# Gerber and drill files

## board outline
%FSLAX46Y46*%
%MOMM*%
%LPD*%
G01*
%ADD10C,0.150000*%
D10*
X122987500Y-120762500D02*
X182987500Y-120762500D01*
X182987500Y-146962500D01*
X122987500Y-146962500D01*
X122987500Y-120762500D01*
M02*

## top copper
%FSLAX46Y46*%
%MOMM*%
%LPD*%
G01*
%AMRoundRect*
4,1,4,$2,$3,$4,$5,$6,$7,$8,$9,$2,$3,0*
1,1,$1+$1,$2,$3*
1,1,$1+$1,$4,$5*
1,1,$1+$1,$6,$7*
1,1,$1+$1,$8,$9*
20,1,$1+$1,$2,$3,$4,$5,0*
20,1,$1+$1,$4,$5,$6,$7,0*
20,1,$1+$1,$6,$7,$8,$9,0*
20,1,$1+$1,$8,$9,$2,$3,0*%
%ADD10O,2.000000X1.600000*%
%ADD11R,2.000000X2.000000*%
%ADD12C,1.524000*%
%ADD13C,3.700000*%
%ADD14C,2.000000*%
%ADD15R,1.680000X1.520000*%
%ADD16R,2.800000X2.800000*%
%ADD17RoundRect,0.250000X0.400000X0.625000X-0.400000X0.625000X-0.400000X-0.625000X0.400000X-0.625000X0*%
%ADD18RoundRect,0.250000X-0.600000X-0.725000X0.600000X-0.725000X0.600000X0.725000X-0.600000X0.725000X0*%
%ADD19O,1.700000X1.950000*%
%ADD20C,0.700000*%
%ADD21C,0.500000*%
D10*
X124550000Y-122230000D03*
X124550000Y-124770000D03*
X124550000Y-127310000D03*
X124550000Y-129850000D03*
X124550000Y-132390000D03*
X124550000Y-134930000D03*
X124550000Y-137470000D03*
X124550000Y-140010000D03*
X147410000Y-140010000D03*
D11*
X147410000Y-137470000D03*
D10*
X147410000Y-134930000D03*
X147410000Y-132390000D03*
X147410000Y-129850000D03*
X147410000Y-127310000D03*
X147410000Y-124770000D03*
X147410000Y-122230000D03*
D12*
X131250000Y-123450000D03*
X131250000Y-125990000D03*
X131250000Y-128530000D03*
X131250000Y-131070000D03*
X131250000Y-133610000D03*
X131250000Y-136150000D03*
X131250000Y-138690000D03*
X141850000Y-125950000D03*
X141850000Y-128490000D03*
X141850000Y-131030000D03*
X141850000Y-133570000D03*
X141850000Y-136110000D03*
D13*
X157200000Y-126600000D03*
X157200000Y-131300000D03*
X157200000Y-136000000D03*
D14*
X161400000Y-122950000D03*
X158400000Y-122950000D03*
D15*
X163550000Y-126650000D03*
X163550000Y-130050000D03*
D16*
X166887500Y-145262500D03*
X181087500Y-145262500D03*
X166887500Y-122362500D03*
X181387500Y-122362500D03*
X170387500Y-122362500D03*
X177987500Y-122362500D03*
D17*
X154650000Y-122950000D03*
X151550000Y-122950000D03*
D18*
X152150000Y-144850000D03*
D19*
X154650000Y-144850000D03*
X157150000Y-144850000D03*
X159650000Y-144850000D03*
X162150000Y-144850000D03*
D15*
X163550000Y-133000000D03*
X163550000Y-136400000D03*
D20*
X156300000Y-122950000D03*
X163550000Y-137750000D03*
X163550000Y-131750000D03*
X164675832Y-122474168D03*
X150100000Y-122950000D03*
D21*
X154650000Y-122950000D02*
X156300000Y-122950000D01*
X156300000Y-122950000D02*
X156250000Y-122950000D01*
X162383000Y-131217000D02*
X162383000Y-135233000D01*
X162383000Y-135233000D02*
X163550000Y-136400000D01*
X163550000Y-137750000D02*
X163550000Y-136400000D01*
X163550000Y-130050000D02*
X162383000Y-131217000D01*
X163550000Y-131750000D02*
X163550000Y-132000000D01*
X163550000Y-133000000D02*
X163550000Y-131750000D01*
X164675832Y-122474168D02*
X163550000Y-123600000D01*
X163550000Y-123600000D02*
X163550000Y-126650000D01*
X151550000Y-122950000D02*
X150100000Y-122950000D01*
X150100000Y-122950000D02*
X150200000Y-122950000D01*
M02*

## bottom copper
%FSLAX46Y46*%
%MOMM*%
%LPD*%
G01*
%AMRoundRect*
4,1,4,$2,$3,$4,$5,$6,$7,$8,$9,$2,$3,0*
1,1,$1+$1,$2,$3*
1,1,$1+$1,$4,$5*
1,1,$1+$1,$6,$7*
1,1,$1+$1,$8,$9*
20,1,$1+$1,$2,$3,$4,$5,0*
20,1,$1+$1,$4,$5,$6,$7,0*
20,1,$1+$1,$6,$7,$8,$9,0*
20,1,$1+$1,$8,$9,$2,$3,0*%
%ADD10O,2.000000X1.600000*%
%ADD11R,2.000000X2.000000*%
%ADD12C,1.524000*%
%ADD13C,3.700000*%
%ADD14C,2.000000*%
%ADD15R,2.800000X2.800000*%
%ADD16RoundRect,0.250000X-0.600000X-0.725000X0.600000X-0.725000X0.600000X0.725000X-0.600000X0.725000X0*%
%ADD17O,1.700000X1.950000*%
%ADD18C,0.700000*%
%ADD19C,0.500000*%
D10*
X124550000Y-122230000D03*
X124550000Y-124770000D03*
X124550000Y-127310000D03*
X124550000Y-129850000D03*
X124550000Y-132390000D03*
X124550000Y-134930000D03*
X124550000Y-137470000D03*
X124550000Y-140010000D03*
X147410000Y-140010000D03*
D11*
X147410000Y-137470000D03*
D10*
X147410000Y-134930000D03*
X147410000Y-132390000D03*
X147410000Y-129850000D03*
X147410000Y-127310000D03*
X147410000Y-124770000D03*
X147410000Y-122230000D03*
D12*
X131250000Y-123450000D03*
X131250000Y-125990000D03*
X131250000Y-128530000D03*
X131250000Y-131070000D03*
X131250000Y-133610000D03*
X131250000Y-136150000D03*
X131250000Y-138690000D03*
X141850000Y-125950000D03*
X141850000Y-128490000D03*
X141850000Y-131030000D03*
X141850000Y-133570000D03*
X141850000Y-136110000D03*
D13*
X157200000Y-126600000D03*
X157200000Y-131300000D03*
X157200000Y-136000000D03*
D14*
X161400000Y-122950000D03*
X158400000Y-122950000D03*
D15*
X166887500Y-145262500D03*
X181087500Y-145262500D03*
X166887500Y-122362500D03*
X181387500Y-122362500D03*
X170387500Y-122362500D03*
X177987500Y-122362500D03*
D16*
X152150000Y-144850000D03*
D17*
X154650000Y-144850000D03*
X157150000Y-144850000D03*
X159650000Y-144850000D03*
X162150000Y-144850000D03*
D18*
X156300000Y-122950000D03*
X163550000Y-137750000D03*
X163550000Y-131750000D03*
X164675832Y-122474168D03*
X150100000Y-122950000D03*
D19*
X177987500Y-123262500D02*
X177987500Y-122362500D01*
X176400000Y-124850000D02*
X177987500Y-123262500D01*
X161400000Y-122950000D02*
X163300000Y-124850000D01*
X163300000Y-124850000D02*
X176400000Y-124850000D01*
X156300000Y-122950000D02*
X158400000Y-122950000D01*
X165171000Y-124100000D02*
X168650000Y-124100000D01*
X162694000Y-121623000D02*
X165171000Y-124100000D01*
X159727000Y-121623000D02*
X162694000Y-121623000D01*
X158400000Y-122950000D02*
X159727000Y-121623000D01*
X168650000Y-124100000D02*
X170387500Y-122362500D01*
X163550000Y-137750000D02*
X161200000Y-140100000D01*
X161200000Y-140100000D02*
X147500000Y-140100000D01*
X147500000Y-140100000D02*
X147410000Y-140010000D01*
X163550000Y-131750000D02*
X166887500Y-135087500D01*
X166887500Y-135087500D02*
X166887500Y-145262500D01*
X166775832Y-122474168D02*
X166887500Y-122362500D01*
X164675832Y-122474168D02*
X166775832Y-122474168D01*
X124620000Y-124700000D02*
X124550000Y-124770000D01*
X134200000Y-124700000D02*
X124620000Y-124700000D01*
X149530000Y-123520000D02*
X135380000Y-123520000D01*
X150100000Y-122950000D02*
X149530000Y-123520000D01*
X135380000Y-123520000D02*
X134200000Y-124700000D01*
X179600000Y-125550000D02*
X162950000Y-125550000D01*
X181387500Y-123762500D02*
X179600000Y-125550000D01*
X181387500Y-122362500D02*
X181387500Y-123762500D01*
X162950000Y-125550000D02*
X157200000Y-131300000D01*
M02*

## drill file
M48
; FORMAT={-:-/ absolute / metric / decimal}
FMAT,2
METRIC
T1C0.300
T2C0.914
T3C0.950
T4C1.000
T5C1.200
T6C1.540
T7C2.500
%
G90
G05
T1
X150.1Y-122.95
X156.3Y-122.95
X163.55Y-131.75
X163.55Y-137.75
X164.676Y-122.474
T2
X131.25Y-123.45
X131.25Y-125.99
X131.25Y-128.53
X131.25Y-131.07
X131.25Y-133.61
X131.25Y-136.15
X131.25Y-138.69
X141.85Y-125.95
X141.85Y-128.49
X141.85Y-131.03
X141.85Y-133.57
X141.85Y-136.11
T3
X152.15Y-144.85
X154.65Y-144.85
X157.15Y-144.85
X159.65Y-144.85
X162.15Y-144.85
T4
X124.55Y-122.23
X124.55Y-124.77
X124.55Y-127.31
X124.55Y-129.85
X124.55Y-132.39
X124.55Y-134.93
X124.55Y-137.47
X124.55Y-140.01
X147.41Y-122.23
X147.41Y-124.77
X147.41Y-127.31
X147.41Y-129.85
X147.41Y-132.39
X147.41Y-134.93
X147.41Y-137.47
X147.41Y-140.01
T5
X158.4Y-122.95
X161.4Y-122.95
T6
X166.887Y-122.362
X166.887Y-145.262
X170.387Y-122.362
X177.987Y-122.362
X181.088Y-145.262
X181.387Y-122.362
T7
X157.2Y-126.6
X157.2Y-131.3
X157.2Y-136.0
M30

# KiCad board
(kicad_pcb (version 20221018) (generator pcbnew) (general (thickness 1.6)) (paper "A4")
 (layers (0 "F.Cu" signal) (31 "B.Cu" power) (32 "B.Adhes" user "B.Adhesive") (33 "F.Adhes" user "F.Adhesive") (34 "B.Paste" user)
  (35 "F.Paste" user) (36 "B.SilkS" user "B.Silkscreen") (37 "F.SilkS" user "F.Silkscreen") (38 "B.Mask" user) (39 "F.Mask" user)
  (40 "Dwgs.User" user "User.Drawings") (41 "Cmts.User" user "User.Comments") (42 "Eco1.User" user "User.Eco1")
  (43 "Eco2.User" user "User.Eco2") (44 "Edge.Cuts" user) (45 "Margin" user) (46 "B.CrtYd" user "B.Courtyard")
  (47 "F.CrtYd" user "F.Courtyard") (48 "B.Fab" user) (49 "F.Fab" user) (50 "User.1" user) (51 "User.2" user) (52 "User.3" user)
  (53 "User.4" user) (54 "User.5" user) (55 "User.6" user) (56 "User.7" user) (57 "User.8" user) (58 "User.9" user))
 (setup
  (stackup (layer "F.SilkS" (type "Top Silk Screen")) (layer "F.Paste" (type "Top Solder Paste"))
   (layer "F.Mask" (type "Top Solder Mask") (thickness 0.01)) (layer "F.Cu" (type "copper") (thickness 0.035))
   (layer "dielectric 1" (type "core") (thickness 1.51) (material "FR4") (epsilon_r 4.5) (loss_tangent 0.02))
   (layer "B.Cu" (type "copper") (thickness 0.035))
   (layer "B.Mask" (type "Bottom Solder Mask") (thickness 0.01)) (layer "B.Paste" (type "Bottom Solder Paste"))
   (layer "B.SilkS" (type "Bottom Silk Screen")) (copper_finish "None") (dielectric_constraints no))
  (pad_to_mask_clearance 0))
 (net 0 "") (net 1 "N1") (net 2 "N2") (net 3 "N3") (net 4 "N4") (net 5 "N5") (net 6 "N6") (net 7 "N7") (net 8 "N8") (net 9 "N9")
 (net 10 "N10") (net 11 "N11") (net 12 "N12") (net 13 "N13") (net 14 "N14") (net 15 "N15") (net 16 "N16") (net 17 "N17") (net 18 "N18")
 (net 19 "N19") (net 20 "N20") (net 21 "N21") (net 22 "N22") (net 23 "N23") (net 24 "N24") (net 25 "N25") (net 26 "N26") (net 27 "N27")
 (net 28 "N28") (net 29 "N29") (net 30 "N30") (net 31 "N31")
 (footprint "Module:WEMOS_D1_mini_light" (layer "F.Cu") (at 124.55 122.23)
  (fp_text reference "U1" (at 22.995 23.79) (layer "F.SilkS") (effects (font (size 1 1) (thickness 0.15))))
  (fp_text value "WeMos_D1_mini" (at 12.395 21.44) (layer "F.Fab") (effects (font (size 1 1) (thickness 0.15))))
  (pad "1" thru_hole oval (at 0 0) (size 2 1.6) (drill 1) (layers "*.Cu" "*.Mask") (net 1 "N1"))
  (pad "2" thru_hole oval (at 0 2.54) (size 2 1.6) (drill 1) (layers "*.Cu" "*.Mask") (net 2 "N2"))
  (pad "3" thru_hole oval (at 0 5.08) (size 2 1.6) (drill 1) (layers "*.Cu" "*.Mask") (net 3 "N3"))
  (pad "4" thru_hole oval (at 0 7.62) (size 2 1.6) (drill 1) (layers "*.Cu" "*.Mask") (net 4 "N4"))
  (pad "5" thru_hole oval (at 0 10.16) (size 2 1.6) (drill 1) (layers "*.Cu" "*.Mask") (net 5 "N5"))
  (pad "6" thru_hole oval (at 0 12.7) (size 2 1.6) (drill 1) (layers "*.Cu" "*.Mask") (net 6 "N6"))
  (pad "7" thru_hole oval (at 0 15.24) (size 2 1.6) (drill 1) (layers "*.Cu" "*.Mask") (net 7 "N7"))
  (pad "8" thru_hole oval (at 0 17.78) (size 2 1.6) (drill 1) (layers "*.Cu" "*.Mask") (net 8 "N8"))
  (pad "9" thru_hole oval (at 22.86 17.78) (size 2 1.6) (drill 1) (layers "*.Cu" "*.Mask") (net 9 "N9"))
  (pad "10" thru_hole rect (at 22.86 15.24) (size 2 2) (drill 1) (layers "*.Cu" "*.Mask") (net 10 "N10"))
  (pad "11" thru_hole oval (at 22.86 12.7) (size 2 1.6) (drill 1) (layers "*.Cu" "*.Mask") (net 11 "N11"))
  (pad "12" thru_hole oval (at 22.86 10.16) (size 2 1.6) (drill 1) (layers "*.Cu" "*.Mask") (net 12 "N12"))
  (pad "13" thru_hole oval (at 22.86 7.62) (size 2 1.6) (drill 1) (layers "*.Cu" "*.Mask") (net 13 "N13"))
  (pad "14" thru_hole oval (at 22.86 5.08) (size 2 1.6) (drill 1) (layers "*.Cu" "*.Mask") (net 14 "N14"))
  (pad "15" thru_hole oval (at 22.86 2.54) (size 2 1.6) (drill 1) (layers "*.Cu" "*.Mask") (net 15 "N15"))
  (pad "16" thru_hole oval (at 22.86 0) (size 2 1.6) (drill 1) (layers "*.Cu" "*.Mask") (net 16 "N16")))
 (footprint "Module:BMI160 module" (layer "F.Cu") (at 129.975 122.075)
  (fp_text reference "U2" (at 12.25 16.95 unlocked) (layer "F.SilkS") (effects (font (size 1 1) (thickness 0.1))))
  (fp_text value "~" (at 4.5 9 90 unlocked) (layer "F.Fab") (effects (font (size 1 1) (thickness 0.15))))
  (pad "1" thru_hole circle (at 1.275 1.375) (size 1.524 1.524) (drill 0.914) (layers "*.Cu" "*.Mask") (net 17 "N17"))
  (pad "2" thru_hole circle (at 1.275 3.915) (size 1.524 1.524) (drill 0.914) (layers "*.Cu" "*.Mask") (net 8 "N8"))
  (pad "3" thru_hole circle (at 1.275 6.455) (size 1.524 1.524) (drill 0.914) (layers "*.Cu" "*.Mask") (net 10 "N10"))
  (pad "4" thru_hole circle (at 1.275 8.995) (size 1.524 1.524) (drill 0.914) (layers "*.Cu" "*.Mask") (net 14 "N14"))
  (pad "5" thru_hole circle (at 1.275 11.535) (size 1.524 1.524) (drill 0.914) (layers "*.Cu" "*.Mask") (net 13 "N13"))
  (pad "6" thru_hole circle (at 1.275 14.075) (size 1.524 1.524) (drill 0.914) (layers "*.Cu" "*.Mask") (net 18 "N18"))
  (pad "7" thru_hole circle (at 1.275 16.615) (size 1.524 1.524) (drill 0.914) (layers "*.Cu" "*.Mask") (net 10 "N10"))
  (pad "8" thru_hole circle (at 11.875 3.875) (size 1.524 1.524) (drill 0.914) (layers "*.Cu" "*.Mask") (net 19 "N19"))
  (pad "9" thru_hole circle (at 11.875 6.415) (size 1.524 1.524) (drill 0.914) (layers "*.Cu" "*.Mask") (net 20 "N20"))
  (pad "10" thru_hole circle (at 11.875 8.955) (size 1.524 1.524) (drill 0.914) (layers "*.Cu" "*.Mask") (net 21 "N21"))
  (pad "11" thru_hole circle (at 11.875 11.495) (size 1.524 1.524) (drill 0.914) (layers "*.Cu" "*.Mask") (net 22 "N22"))
  (pad "12" thru_hole circle (at 11.875 14.035) (size 1.524 1.524) (drill 0.914) (layers "*.Cu" "*.Mask") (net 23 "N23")))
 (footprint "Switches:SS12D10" (layer "F.Cu") (at 157.1 131.25 -90)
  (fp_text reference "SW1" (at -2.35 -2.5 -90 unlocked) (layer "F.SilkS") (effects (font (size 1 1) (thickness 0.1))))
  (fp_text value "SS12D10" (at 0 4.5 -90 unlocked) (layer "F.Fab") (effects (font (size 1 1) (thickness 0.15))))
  (pad "1" thru_hole circle (at -4.65 -0.1 270) (size 3.7 3.7) (drill 2.5) (layers "*.Cu" "*.Mask") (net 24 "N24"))
  (pad "2" thru_hole circle (at 0.05 -0.1 270) (size 3.7 3.7) (drill 2.5) (layers "*.Cu" "*.Mask") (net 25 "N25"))
  (pad "3" thru_hole circle (at 4.75 -0.1 270) (size 3.7 3.7) (drill 2.5) (layers "*.Cu" "*.Mask") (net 10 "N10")))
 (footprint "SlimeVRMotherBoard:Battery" (layer "F.Cu") (at 159.9 122.95 -90)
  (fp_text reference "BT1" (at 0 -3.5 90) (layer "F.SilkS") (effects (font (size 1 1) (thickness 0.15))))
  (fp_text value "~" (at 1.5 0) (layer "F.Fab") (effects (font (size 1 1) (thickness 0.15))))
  (pad "1" thru_hole circle (at 0 -1.5 270) (size 2 2) (drill 1.2) (layers "*.Cu" "*.Mask") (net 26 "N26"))
  (pad "2" thru_hole circle (at 0 1.5 270) (size 2 2) (drill 1.2) (layers "*.Cu" "*.Mask") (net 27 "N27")))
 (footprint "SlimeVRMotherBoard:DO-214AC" (layer "F.Cu") (at 163.55 128.35 90) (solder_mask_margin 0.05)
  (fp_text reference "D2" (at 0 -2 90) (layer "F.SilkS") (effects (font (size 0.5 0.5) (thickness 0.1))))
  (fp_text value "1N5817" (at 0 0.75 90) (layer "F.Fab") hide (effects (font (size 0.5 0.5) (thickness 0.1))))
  (pad "A" smd rect (at 1.7 0 90) (size 1.52 1.68) (layers "F.Cu" "F.Paste" "F.Mask") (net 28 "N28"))
  (pad "C" smd rect (at -1.7 0 90) (size 1.52 1.68) (layers "F.Cu" "F.Paste" "F.Mask") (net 9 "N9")))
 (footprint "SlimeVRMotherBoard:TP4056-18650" (layer "F.Cu") (at 165.1875 146.9625 90)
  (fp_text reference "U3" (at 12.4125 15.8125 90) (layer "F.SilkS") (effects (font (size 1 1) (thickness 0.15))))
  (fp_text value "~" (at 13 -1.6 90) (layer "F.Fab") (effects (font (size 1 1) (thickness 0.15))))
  (pad "1" thru_hole rect (at 1.7 1.7 90) (size 2.8 2.8) (drill 1.54) (layers "*.Cu" "*.Mask") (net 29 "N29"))
  (pad "2" thru_hole rect (at 1.7 15.9 90) (size 2.8 2.8) (drill 1.54) (layers "*.Cu" "*.Mask") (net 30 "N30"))
  (pad "3" thru_hole rect (at 24.6 1.7 90) (size 2.8 2.8) (drill 1.54) (layers "*.Cu" "*.Mask") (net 28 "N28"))
  (pad "4" thru_hole rect (at 24.6 16.2 90) (size 2.8 2.8) (drill 1.54) (layers "*.Cu" "*.Mask") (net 25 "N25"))
  (pad "5" thru_hole rect (at 24.6 5.2 90) (size 2.8 2.8) (drill 1.54) (layers "*.Cu" "*.Mask") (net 27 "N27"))
  (pad "6" thru_hole rect (at 24.6 12.8 90) (size 2.8 2.8) (drill 1.54) (layers "*.Cu" "*.Mask") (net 26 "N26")))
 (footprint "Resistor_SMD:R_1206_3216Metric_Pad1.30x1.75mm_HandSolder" (layer "F.Cu") (at 153.1 122.95 180)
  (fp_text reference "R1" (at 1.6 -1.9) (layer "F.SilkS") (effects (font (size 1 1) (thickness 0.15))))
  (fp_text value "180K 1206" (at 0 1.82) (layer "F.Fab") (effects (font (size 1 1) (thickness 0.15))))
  (pad "1" smd roundrect (at -1.55 0 180) (size 1.3 1.75) (layers "F.Cu" "F.Paste" "F.Mask") (roundrect_rratio 0.192308) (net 27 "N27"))
  (pad "2" smd roundrect (at 1.55 0 180) (size 1.3 1.75) (layers "F.Cu" "F.Paste" "F.Mask") (roundrect_rratio 0.192308) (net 2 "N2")))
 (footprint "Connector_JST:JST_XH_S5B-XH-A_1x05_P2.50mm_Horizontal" (layer "F.Cu") (at 152.15 144.85)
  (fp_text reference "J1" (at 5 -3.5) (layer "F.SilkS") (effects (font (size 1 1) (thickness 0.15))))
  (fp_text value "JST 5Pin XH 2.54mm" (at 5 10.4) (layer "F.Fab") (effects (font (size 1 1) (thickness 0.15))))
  (pad "1" thru_hole roundrect (at 0 0) (size 1.7 1.95) (drill 0.95) (layers "*.Cu" "*.Mask") (roundrect_rratio 0.147059) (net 13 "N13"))
  (pad "2" thru_hole oval (at 2.5 0) (size 1.7 1.95) (drill 0.95) (layers "*.Cu" "*.Mask") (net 8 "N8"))
  (pad "3" thru_hole oval (at 5 0) (size 1.7 1.95) (drill 0.95) (layers "*.Cu" "*.Mask") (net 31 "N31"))
  (pad "4" thru_hole oval (at 7.5 0) (size 1.7 1.95) (drill 0.95) (layers "*.Cu" "*.Mask") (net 10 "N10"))
  (pad "5" thru_hole oval (at 10 0) (size 1.7 1.95) (drill 0.95) (layers "*.Cu" "*.Mask") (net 14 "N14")))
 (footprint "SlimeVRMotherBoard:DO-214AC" (layer "F.Cu") (at 163.55 134.7 90) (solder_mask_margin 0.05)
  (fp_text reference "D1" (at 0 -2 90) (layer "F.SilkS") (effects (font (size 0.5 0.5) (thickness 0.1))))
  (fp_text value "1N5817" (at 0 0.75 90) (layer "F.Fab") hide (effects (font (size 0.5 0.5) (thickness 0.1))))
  (pad "A" smd rect (at 1.7 0 90) (size 1.52 1.68) (layers "F.Cu" "F.Paste" "F.Mask") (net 29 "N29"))
  (pad "C" smd rect (at -1.7 0 90) (size 1.52 1.68) (layers "F.Cu" "F.Paste" "F.Mask") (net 9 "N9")))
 (gr_rect (start 122.9875 120.7625) (end 182.9875 146.9625) (stroke (width 0.15) (type default)) (fill none) (layer "Edge.Cuts"))
 (segment (start 177.9875 123.2625) (end 177.9875 122.3625) (width 0.5) (layer "B.Cu") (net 26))
 (segment (start 176.4 124.85) (end 177.9875 123.2625) (width 0.5) (layer "B.Cu") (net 26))
 (segment (start 161.4 122.95) (end 163.3 124.85) (width 0.5) (layer "B.Cu") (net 26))
 (segment (start 163.3 124.85) (end 176.4 124.85) (width 0.5) (layer "B.Cu") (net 26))
 (segment (start 154.65 122.95) (end 156.3 122.95) (width 0.5) (layer "F.Cu") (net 27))
 (segment (start 156.3 122.95) (end 156.25 122.95) (width 0.5) (layer "F.Cu") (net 27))
 (via (at 156.3 122.95) (size 0.7) (drill 0.3) (layers "F.Cu" "B.Cu") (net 27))
 (segment (start 156.3 122.95) (end 158.4 122.95) (width 0.5) (layer "B.Cu") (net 27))
 (segment (start 165.171 124.1) (end 168.65 124.1) (width 0.5) (layer "B.Cu") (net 27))
 (segment (start 162.694 121.623) (end 165.171 124.1) (width 0.5) (layer "B.Cu") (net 27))
 (segment (start 159.727 121.623) (end 162.694 121.623) (width 0.5) (layer "B.Cu") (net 27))
 (segment (start 158.4 122.95) (end 159.727 121.623) (width 0.5) (layer "B.Cu") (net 27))
 (segment (start 168.65 124.1) (end 170.3875 122.3625) (width 0.5) (layer "B.Cu") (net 27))
 (segment (start 162.383 131.217) (end 162.383 135.233) (width 0.5) (layer "F.Cu") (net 9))
 (segment (start 162.383 135.233) (end 163.55 136.4) (width 0.5) (layer "F.Cu") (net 9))
 (segment (start 163.55 137.75) (end 163.55 136.4) (width 0.5) (layer "F.Cu") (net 9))
 (segment (start 163.55 130.05) (end 162.383 131.217) (width 0.5) (layer "F.Cu") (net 9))
 (via (at 163.55 137.75) (size 0.7) (drill 0.3) (layers "F.Cu" "B.Cu") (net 9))
 (segment (start 163.55 137.75) (end 161.2 140.1) (width 0.5) (layer "B.Cu") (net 9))
 (segment (start 161.2 140.1) (end 147.5 140.1) (width 0.5) (layer "B.Cu") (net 9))
 (segment (start 147.5 140.1) (end 147.41 140.01) (width 0.5) (layer "B.Cu") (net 9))
 (segment (start 163.55 131.75) (end 163.55 132) (width 0.5) (layer "F.Cu") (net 29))
 (segment (start 163.55 133) (end 163.55 131.75) (width 0.5) (layer "F.Cu") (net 29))
 (via (at 163.55 131.75) (size 0.7) (drill 0.3) (layers "F.Cu" "B.Cu") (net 29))
 (segment (start 163.55 131.75) (end 166.8875 135.0875) (width 0.5) (layer "B.Cu") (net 29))
 (segment (start 166.8875 135.0875) (end 166.8875 145.2625) (width 0.5) (layer "B.Cu") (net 29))
 (segment (start 164.675832 122.474168) (end 163.55 123.6) (width 0.5) (layer "F.Cu") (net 28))
 (segment (start 163.55 123.6) (end 163.55 126.65) (width 0.5) (layer "F.Cu") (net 28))
 (via (at 164.675832 122.474168) (size 0.7) (drill 0.3) (layers "F.Cu" "B.Cu") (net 28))
 (segment (start 166.775832 122.474168) (end 166.8875 122.3625) (width 0.5) (layer "B.Cu") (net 28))
 (segment (start 164.675832 122.474168) (end 166.775832 122.474168) (width 0.5) (layer "B.Cu") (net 28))
 (segment (start 151.55 122.95) (end 150.1 122.95) (width 0.5) (layer "F.Cu") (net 2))
 (segment (start 150.1 122.95) (end 150.2 122.95) (width 0.5) (layer "F.Cu") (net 2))
 (via (at 150.1 122.95) (size 0.7) (drill 0.3) (layers "F.Cu" "B.Cu") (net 2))
 (segment (start 124.62 124.7) (end 124.55 124.77) (width 0.5) (layer "B.Cu") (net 2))
 (segment (start 134.2 124.7) (end 124.62 124.7) (width 0.5) (layer "B.Cu") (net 2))
 (segment (start 149.53 123.52) (end 135.38 123.52) (width 0.5) (layer "B.Cu") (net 2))
 (segment (start 150.1 122.95) (end 149.53 123.52) (width 0.5) (layer "B.Cu") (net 2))
 (segment (start 135.38 123.52) (end 134.2 124.7) (width 0.5) (layer "B.Cu") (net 2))
 (segment (start 179.6 125.55) (end 162.95 125.55) (width 0.5) (layer "B.Cu") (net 25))
 (segment (start 181.3875 123.7625) (end 179.6 125.55) (width 0.5) (layer "B.Cu") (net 25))
 (segment (start 181.3875 122.3625) (end 181.3875 123.7625) (width 0.5) (layer "B.Cu") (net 25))
 (segment (start 162.95 125.55) (end 157.2 131.3) (width 0.5) (layer "B.Cu") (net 25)))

